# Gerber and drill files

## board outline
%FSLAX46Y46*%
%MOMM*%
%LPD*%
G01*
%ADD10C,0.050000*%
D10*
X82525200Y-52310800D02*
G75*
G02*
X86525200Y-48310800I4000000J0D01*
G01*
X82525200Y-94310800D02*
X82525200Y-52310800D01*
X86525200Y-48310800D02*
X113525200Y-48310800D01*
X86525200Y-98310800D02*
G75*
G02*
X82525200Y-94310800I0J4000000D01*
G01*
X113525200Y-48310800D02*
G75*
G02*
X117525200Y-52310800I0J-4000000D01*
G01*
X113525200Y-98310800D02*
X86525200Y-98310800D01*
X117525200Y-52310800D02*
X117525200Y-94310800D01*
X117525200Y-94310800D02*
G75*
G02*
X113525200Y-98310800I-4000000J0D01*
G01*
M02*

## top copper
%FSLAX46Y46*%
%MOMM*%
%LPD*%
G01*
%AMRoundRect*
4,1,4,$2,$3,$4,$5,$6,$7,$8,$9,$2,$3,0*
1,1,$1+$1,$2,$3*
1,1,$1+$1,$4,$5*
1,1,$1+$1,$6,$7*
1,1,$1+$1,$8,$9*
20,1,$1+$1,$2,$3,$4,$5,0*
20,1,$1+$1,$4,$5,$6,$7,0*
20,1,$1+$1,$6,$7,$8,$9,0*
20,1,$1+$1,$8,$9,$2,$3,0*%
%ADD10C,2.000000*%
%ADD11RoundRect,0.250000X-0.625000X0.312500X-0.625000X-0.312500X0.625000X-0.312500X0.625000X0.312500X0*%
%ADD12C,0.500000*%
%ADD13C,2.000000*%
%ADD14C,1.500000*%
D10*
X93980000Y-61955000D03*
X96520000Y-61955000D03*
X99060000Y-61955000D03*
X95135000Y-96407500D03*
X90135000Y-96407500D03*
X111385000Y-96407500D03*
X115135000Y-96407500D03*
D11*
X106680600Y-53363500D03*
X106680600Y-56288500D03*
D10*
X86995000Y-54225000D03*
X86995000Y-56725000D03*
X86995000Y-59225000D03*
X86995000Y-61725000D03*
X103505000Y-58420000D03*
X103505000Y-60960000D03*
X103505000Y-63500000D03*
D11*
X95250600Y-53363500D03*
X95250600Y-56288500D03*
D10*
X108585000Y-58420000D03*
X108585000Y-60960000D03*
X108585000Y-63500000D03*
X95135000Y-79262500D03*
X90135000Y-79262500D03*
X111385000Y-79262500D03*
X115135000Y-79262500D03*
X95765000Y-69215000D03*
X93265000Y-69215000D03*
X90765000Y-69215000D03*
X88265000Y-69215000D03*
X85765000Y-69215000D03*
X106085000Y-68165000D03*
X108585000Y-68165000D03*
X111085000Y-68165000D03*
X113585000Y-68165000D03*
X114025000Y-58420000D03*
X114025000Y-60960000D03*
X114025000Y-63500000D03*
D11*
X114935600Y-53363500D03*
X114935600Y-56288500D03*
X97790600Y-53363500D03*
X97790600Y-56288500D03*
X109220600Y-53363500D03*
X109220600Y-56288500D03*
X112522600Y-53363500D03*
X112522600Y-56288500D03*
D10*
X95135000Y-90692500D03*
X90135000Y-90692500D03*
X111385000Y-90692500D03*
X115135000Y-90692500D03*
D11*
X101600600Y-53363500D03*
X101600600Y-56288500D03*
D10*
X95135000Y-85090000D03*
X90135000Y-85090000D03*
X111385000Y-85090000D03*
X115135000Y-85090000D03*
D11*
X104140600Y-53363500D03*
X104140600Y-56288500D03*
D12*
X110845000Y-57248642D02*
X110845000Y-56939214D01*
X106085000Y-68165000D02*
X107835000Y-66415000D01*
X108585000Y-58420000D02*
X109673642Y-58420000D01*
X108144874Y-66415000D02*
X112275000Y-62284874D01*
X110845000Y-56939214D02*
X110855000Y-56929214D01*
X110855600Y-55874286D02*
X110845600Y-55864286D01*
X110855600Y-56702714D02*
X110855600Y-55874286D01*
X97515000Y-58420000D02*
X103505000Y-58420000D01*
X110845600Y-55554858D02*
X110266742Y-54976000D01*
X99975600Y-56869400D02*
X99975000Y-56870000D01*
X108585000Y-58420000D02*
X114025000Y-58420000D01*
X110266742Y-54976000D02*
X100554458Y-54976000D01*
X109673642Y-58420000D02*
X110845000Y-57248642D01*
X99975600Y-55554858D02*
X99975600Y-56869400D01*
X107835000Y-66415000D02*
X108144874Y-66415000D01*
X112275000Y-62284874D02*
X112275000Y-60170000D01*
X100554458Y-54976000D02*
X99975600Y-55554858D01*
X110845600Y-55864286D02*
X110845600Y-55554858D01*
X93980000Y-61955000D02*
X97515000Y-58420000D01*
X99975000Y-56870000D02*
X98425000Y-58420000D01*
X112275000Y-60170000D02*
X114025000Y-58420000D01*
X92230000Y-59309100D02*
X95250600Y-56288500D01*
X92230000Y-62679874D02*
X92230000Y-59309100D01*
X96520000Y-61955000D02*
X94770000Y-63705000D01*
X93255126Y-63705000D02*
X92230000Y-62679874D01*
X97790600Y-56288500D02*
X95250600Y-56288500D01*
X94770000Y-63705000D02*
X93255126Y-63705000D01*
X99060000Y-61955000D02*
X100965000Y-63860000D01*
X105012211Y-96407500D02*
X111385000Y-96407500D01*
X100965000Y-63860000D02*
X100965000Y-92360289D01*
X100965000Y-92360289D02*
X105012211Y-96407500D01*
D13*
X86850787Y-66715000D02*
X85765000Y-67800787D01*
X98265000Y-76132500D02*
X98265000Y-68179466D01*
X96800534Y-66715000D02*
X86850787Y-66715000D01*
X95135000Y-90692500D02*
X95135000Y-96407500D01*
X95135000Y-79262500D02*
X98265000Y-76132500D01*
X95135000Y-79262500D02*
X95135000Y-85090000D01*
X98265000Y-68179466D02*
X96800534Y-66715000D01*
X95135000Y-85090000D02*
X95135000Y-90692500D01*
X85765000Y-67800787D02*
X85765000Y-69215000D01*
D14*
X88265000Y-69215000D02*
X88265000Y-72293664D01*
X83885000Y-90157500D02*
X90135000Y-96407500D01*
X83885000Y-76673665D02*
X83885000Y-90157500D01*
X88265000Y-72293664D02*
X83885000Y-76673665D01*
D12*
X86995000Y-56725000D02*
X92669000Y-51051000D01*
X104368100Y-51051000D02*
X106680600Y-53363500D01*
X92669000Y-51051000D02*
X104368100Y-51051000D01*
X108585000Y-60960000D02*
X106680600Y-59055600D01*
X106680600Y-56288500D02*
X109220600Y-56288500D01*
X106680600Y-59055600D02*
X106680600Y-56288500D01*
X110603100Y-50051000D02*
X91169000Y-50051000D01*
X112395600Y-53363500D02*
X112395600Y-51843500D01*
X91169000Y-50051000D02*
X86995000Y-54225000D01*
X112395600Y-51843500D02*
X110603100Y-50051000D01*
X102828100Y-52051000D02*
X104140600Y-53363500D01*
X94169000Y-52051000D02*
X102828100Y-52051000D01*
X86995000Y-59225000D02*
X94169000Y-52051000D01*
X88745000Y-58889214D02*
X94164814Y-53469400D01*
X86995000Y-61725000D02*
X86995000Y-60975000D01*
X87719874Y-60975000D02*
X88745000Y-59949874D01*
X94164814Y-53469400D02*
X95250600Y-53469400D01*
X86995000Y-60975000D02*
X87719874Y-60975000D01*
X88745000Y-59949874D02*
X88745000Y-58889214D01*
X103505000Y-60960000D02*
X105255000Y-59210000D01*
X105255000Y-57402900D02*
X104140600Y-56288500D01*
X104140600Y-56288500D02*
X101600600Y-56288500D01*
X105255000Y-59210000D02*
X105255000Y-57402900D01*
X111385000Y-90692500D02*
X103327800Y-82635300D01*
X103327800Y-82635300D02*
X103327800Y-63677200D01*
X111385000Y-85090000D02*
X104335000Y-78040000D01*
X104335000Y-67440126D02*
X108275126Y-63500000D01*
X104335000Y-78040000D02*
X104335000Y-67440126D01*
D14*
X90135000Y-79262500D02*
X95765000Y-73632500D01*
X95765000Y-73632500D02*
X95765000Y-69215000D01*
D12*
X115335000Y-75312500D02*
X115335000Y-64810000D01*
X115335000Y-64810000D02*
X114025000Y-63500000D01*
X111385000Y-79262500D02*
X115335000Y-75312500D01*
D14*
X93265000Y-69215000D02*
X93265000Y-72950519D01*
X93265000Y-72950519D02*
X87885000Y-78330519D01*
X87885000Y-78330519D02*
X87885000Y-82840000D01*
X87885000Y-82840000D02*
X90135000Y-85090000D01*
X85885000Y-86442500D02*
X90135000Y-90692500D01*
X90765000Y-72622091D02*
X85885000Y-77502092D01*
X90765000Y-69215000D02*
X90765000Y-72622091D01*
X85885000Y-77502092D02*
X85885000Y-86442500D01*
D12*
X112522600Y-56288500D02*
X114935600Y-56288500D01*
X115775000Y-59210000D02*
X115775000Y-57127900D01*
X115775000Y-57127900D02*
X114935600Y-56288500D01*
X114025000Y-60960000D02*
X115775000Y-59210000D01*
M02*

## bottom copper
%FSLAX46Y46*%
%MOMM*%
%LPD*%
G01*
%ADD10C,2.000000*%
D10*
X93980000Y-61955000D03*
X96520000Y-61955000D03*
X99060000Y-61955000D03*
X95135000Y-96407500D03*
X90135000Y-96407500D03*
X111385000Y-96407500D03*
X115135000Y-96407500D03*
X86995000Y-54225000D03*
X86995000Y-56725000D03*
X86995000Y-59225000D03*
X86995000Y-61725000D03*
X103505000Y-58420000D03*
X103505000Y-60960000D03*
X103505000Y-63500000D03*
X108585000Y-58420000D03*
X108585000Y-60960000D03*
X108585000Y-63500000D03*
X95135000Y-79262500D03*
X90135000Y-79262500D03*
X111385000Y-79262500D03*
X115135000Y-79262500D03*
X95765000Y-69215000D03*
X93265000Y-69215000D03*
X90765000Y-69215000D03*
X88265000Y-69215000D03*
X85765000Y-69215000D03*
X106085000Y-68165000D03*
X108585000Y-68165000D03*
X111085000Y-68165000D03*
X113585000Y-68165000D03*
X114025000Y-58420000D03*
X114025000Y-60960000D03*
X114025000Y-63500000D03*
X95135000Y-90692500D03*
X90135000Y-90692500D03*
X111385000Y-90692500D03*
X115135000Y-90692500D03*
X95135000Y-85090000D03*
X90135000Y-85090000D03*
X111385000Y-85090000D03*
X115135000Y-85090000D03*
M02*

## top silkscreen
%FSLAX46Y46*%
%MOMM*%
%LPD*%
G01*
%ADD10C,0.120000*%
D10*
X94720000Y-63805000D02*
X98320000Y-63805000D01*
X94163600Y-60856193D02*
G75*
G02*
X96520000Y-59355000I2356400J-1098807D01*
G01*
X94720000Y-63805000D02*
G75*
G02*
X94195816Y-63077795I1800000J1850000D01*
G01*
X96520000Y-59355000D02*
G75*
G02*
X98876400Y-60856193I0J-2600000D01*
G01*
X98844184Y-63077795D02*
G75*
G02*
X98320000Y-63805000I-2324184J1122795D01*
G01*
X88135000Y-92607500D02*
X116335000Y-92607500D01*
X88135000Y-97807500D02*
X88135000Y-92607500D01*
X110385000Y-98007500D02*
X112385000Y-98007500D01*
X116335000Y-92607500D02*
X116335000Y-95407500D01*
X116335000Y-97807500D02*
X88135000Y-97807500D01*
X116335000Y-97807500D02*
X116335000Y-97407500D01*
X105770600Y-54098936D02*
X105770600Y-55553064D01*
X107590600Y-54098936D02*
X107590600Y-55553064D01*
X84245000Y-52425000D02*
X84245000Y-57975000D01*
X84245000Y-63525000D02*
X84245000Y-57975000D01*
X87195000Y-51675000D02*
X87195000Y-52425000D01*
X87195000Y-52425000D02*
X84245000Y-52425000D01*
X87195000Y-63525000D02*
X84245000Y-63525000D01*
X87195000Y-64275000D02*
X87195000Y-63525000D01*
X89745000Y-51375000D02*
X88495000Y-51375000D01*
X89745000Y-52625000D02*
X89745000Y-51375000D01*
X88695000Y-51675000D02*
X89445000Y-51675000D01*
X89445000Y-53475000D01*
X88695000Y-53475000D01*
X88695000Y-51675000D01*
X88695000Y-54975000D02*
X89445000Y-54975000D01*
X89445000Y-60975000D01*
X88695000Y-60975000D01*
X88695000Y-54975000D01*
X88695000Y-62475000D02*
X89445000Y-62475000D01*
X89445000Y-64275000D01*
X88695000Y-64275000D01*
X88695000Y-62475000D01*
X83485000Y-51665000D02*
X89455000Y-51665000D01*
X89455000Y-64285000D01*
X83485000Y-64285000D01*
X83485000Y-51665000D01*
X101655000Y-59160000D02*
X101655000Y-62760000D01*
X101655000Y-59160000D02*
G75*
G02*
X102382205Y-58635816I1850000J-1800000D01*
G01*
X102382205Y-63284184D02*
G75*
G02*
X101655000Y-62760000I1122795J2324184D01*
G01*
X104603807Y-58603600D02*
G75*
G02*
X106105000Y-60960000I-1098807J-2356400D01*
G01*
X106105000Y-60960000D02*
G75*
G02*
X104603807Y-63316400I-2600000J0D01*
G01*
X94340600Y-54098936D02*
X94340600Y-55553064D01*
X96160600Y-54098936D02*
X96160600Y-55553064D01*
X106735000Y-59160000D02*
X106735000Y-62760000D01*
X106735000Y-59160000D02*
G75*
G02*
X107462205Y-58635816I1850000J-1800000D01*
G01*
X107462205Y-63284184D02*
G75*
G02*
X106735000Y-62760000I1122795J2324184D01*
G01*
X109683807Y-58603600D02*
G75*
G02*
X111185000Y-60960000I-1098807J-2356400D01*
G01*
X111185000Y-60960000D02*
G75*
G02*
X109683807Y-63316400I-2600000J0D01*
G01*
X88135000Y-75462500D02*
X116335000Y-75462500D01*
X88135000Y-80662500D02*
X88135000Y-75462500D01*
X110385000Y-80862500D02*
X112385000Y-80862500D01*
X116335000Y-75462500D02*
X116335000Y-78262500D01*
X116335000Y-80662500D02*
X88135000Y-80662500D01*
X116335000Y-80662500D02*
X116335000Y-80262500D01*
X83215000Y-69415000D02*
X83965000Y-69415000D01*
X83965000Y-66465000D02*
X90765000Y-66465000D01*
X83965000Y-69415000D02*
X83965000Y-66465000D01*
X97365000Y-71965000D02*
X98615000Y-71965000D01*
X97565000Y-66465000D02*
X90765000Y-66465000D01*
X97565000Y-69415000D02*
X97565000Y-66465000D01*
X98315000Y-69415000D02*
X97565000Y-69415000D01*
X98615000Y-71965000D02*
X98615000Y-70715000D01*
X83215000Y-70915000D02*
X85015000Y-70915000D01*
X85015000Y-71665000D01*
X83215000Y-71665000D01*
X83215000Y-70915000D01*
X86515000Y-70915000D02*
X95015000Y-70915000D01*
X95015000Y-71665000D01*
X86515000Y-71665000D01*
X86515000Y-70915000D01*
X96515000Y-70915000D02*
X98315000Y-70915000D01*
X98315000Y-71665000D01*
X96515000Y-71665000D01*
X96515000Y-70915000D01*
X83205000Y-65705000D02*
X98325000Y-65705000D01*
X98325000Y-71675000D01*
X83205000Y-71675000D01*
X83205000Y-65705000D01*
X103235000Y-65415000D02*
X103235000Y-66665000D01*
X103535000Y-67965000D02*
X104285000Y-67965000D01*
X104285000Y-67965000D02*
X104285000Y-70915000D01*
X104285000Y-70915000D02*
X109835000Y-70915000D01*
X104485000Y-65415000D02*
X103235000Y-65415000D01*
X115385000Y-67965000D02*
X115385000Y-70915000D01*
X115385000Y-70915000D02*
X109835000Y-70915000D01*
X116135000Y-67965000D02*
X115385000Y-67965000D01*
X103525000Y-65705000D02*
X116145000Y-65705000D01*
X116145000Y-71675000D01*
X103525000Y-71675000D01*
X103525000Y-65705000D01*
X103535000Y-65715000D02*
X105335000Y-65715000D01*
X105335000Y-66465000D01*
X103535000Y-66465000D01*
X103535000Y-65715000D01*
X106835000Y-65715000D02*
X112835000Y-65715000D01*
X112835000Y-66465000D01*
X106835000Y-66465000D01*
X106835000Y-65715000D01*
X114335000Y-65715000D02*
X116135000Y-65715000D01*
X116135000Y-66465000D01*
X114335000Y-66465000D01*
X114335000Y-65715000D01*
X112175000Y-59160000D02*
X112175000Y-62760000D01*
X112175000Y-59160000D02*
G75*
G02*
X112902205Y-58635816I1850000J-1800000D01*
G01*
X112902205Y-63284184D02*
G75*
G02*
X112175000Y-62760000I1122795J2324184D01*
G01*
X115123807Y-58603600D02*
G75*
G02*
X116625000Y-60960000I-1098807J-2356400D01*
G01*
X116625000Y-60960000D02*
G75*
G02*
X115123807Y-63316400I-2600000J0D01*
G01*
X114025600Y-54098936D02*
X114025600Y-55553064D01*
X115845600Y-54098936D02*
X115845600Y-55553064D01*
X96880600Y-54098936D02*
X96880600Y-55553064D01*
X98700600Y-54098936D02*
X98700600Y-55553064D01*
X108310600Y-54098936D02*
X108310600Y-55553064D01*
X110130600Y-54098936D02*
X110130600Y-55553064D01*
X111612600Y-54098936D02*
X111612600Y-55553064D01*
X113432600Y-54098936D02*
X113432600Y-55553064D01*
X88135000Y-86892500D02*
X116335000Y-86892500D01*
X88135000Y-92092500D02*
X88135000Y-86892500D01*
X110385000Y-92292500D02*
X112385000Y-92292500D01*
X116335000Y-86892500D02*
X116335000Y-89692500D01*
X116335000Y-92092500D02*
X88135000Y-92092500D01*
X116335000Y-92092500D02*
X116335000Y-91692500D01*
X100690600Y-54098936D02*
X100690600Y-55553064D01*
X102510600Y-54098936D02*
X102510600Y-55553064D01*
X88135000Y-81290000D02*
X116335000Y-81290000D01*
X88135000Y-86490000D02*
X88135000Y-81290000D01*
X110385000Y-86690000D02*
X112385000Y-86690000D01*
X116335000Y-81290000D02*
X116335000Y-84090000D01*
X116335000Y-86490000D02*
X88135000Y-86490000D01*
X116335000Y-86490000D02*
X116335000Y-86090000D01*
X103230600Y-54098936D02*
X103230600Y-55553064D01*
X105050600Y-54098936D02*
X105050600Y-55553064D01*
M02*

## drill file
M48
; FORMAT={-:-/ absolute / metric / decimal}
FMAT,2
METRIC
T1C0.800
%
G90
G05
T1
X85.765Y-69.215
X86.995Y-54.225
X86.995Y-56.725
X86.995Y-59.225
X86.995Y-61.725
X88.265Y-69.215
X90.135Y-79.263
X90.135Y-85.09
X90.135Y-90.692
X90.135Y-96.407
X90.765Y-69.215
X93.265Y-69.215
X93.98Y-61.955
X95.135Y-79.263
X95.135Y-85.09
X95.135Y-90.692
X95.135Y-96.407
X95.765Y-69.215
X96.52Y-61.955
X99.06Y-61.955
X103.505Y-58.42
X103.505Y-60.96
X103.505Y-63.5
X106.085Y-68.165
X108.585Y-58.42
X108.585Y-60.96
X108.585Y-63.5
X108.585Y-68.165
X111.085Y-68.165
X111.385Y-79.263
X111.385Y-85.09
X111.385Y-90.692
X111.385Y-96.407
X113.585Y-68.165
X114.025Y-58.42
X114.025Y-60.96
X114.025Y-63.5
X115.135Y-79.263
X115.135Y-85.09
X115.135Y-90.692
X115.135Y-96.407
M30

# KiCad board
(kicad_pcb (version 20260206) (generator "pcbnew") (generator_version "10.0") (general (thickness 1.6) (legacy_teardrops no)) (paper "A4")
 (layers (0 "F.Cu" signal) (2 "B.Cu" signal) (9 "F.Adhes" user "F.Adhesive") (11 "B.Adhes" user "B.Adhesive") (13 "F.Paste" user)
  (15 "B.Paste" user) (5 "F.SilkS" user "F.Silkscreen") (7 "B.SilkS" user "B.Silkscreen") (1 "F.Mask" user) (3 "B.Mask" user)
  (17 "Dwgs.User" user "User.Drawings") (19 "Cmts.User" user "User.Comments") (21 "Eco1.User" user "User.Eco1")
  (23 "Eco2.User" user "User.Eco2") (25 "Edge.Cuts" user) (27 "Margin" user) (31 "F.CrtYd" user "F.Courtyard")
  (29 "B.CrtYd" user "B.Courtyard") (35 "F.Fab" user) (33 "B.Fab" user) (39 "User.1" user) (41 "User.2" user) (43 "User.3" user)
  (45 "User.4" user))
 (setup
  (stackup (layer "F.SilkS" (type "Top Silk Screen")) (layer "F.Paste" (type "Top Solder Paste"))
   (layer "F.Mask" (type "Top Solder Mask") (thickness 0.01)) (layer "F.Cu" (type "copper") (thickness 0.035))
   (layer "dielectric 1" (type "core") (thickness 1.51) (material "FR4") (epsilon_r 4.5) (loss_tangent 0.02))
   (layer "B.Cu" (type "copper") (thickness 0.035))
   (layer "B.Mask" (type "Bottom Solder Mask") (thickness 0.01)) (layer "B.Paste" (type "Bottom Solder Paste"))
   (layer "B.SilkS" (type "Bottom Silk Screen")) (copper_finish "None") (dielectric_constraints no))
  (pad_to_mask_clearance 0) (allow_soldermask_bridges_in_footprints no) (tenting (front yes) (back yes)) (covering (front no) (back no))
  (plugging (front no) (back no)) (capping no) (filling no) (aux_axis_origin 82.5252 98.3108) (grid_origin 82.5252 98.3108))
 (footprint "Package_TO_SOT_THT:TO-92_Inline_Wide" (layer "F.Cu") (at 93.98 61.955)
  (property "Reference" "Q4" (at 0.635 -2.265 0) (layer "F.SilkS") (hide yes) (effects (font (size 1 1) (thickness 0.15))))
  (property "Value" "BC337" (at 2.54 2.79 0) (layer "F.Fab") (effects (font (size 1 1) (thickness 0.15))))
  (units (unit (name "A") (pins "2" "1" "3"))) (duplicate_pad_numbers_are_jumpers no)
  (fp_line (start 0.74 1.85) (end 4.34 1.85) (stroke (width 0.12) (type solid)) (layer "F.SilkS"))
  (fp_arc (start 0.1836 -1.098807) (mid 1.143021 -2.192817) (end 2.54 -2.6) (stroke (width 0.12) (type solid)) (layer "F.SilkS"))
  (fp_arc (start 0.74 1.85) (mid 0.446097 1.509328) (end 0.215816 1.122795) (stroke (width 0.12) (type solid)) (layer "F.SilkS"))
  (fp_arc (start 2.54 -2.6) (mid 3.936979 -2.192818) (end 4.8964 -1.098807) (stroke (width 0.12) (type solid)) (layer "F.SilkS"))
  (fp_arc (start 4.864184 1.122795) (mid 4.633903 1.509328) (end 4.34 1.85) (stroke (width 0.12) (type solid)) (layer "F.SilkS"))
  (pad "1" thru_hole circle (at 0 0) (size 2 1.5) (drill 0.8) (layers "*.Cu" "*.Mask") (remove_unused_layers no) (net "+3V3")
   (thermal_bridge_angle 90))
  (pad "2" thru_hole circle (at 2.54 0) (size 2 1.5) (drill 0.8) (layers "*.Cu" "*.Mask") (remove_unused_layers no) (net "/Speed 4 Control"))
  (pad "3" thru_hole circle (at 5.08 0) (size 2 1.5) (drill 0.8) (layers "*.Cu" "*.Mask") (remove_unused_layers no) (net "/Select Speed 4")))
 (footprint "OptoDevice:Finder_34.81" (layer "F.Cu") (at 111.385 96.4075 180)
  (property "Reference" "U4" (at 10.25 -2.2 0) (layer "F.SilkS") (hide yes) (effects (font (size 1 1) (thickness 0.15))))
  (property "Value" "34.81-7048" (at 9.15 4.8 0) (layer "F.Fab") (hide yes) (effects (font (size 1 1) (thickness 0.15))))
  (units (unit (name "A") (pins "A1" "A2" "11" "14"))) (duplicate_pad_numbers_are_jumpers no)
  (fp_line (start 23.25 3.8) (end -4.95 3.8) (stroke (width 0.12) (type solid)) (layer "F.SilkS"))
  (fp_line (start 23.25 -1.4) (end 23.25 3.8) (stroke (width 0.12) (type solid)) (layer "F.SilkS"))
  (fp_line (start 1 -1.6) (end -1 -1.6) (stroke (width 0.12) (type solid)) (layer "F.SilkS"))
  (fp_line (start -4.95 3.8) (end -4.95 1) (stroke (width 0.12) (type solid)) (layer "F.SilkS"))
  (fp_line (start -4.95 -1.4) (end 23.25 -1.4) (stroke (width 0.12) (type solid)) (layer "F.SilkS"))
  (fp_line (start -4.95 -1.4) (end -4.95 -1) (stroke (width 0.12) (type solid)) (layer "F.SilkS"))
  (pad "11" thru_hole circle (at 16.25 0 180) (size 2 2.4) (drill 0.8) (layers "*.Cu" "*.Mask") (remove_unused_layers no) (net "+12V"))
  (pad "14" thru_hole circle (at 21.25 0 180) (size 2 2.4) (drill 0.8) (layers "*.Cu" "*.Mask") (remove_unused_layers no) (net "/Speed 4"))
  (pad "A1" thru_hole circle (at 0 0 180) (size 2 2.4) (drill 0.8) (layers "*.Cu" "*.Mask") (remove_unused_layers no)
   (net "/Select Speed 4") (thermal_bridge_angle 90))
  (pad "A2" thru_hole circle (at -3.75 0 180) (size 2 2.4) (drill 0.8) (layers "*.Cu" "*.Mask") (remove_unused_layers no) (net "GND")))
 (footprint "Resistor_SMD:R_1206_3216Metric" (layer "F.Cu") (at 106.6806 54.826 -90)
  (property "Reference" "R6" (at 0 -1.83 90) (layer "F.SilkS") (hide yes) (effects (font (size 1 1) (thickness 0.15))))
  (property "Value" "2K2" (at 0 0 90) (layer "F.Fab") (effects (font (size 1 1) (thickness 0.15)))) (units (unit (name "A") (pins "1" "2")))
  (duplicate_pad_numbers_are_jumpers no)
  (fp_line (start -0.727064 0.91) (end 0.727064 0.91) (stroke (width 0.12) (type solid)) (layer "F.SilkS"))
  (fp_line (start -0.727064 -0.91) (end 0.727064 -0.91) (stroke (width 0.12) (type solid)) (layer "F.SilkS"))
  (pad "1" smd roundrect (at -1.4625 0 270) (size 1.125 1.75) (layers "F.Cu" "F.Mask" "F.Paste") (roundrect_rratio 0.222222) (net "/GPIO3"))
  (pad "2" smd roundrect (at 1.4625 0 270) (size 1.125 1.75) (layers "F.Cu" "F.Mask" "F.Paste") (roundrect_rratio 0.222222)
   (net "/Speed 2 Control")))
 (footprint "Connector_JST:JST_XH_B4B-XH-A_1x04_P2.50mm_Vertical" (layer "F.Cu") (at 86.995 54.225 -90)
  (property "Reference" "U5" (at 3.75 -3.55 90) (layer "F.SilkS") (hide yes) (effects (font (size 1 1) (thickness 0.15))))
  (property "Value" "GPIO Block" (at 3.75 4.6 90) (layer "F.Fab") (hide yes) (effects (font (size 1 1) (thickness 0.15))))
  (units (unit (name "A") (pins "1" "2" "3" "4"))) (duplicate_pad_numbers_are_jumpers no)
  (fp_line (start -1.8 2.75) (end 3.75 2.75) (stroke (width 0.12) (type solid)) (layer "F.SilkS"))
  (fp_line (start 9.3 2.75) (end 3.75 2.75) (stroke (width 0.12) (type solid)) (layer "F.SilkS"))
  (fp_line (start -2.55 -0.2) (end -1.8 -0.2) (stroke (width 0.12) (type solid)) (layer "F.SilkS"))
  (fp_line (start -1.8 -0.2) (end -1.8 2.75) (stroke (width 0.12) (type solid)) (layer "F.SilkS"))
  (fp_line (start 9.3 -0.2) (end 9.3 2.75) (stroke (width 0.12) (type solid)) (layer "F.SilkS"))
  (fp_line (start 10.05 -0.2) (end 9.3 -0.2) (stroke (width 0.12) (type solid)) (layer "F.SilkS"))
  (fp_line (start -2.85 -2.75) (end -2.85 -1.5) (stroke (width 0.12) (type solid)) (layer "F.SilkS"))
  (fp_line (start -1.6 -2.75) (end -2.85 -2.75) (stroke (width 0.12) (type solid)) (layer "F.SilkS"))
  (fp_rect (start -2.55 -2.45) (end -0.75 -1.7) (stroke (width 0.12) (type solid)) (fill no) (layer "F.SilkS"))
  (fp_rect (start 0.75 -2.45) (end 6.75 -1.7) (stroke (width 0.12) (type solid)) (fill no) (layer "F.SilkS"))
  (fp_rect (start 8.25 -2.45) (end 10.05 -1.7) (stroke (width 0.12) (type solid)) (fill no) (layer "F.SilkS"))
  (fp_rect (start -2.56 -2.46) (end 10.06 3.51) (stroke (width 0.12) (type solid)) (fill no) (layer "F.SilkS"))
  (pad "1" thru_hole circle (at 0 0 270) (size 2 1.95) (drill 0.8) (layers "*.Cu" "*.Mask") (remove_unused_layers no) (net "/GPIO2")
   (thermal_bridge_angle 90))
  (pad "2" thru_hole circle (at 2.5 0 270) (size 2 1.95) (drill 0.8) (layers "*.Cu" "*.Mask") (remove_unused_layers no) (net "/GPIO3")
   (thermal_bridge_angle 90))
  (pad "3" thru_hole circle (at 5 0 270) (size 2 1.95) (drill 0.8) (layers "*.Cu" "*.Mask") (remove_unused_layers no) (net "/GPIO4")
   (thermal_bridge_angle 90))
  (pad "4" thru_hole circle (at 7.5 0 270) (size 2 1.95) (drill 0.8) (layers "*.Cu" "*.Mask") (remove_unused_layers no) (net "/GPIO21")
   (thermal_bridge_angle 90)))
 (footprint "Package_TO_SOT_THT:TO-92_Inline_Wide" (layer "F.Cu") (at 103.505 58.42 -90)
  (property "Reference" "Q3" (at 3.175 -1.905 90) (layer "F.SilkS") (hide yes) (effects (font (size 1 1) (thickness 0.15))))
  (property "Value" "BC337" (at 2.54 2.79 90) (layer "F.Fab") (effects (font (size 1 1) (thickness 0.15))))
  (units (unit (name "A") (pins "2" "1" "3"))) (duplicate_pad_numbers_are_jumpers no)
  (fp_line (start 0.74 1.85) (end 4.34 1.85) (stroke (width 0.12) (type solid)) (layer "F.SilkS"))
  (fp_arc (start 0.74 1.85) (mid 0.446097 1.509328) (end 0.215816 1.122795) (stroke (width 0.12) (type solid)) (layer "F.SilkS"))
  (fp_arc (start 4.864184 1.122795) (mid 4.633903 1.509328) (end 4.34 1.85) (stroke (width 0.12) (type solid)) (layer "F.SilkS"))
  (fp_arc (start 0.1836 -1.098807) (mid 1.143021 -2.192817) (end 2.54 -2.6) (stroke (width 0.12) (type solid)) (layer "F.SilkS"))
  (fp_arc (start 2.54 -2.6) (mid 3.936979 -2.192818) (end 4.8964 -1.098807) (stroke (width 0.12) (type solid)) (layer "F.SilkS"))
  (pad "1" thru_hole circle (at 0 0 270) (size 2 1.5) (drill 0.8) (layers "*.Cu" "*.Mask") (remove_unused_layers no) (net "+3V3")
   (thermal_bridge_angle 90))
  (pad "2" thru_hole circle (at 2.54 0 270) (size 2 1.5) (drill 0.8) (layers "*.Cu" "*.Mask") (remove_unused_layers no)
   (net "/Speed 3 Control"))
  (pad "3" thru_hole circle (at 5.08 0 270) (size 2 1.5) (drill 0.8) (layers "*.Cu" "*.Mask") (remove_unused_layers no)
   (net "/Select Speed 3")))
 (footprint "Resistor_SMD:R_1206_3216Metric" (layer "F.Cu") (at 95.2506 54.826 -90)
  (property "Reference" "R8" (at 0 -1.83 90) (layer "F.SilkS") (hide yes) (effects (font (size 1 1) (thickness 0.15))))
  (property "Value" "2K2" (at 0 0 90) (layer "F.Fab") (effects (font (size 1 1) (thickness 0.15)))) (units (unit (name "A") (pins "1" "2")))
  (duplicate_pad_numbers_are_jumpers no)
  (fp_line (start -0.727064 0.91) (end 0.727064 0.91) (stroke (width 0.12) (type solid)) (layer "F.SilkS"))
  (fp_line (start -0.727064 -0.91) (end 0.727064 -0.91) (stroke (width 0.12) (type solid)) (layer "F.SilkS"))
  (pad "1" smd roundrect (at -1.4625 0 270) (size 1.125 1.75) (layers "F.Cu" "F.Mask" "F.Paste") (roundrect_rratio 0.222222) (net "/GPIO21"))
  (pad "2" smd roundrect (at 1.4625 0 270) (size 1.125 1.75) (layers "F.Cu" "F.Mask" "F.Paste") (roundrect_rratio 0.222222)
   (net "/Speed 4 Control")))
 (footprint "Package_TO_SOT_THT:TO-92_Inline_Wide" (layer "F.Cu") (at 108.585 58.42 -90)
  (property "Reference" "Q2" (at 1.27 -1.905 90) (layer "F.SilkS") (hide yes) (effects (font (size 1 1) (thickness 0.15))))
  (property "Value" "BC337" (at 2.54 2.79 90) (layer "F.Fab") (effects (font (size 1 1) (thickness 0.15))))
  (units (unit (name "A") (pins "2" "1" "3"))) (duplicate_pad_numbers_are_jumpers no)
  (fp_line (start 0.74 1.85) (end 4.34 1.85) (stroke (width 0.12) (type solid)) (layer "F.SilkS"))
  (fp_arc (start 0.74 1.85) (mid 0.446097 1.509328) (end 0.215816 1.122795) (stroke (width 0.12) (type solid)) (layer "F.SilkS"))
  (fp_arc (start 4.864184 1.122795) (mid 4.633903 1.509328) (end 4.34 1.85) (stroke (width 0.12) (type solid)) (layer "F.SilkS"))
  (fp_arc (start 0.1836 -1.098807) (mid 1.143021 -2.192817) (end 2.54 -2.6) (stroke (width 0.12) (type solid)) (layer "F.SilkS"))
  (fp_arc (start 2.54 -2.6) (mid 3.936979 -2.192818) (end 4.8964 -1.098807) (stroke (width 0.12) (type solid)) (layer "F.SilkS"))
  (pad "1" thru_hole circle (at 0 0 270) (size 2 1.5) (drill 0.8) (layers "*.Cu" "*.Mask") (remove_unused_layers no) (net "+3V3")
   (thermal_bridge_angle 90))
  (pad "2" thru_hole circle (at 2.54 0 270) (size 2 1.5) (drill 0.8) (layers "*.Cu" "*.Mask") (remove_unused_layers no)
   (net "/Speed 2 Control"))
  (pad "3" thru_hole circle (at 5.08 0 270) (size 2 1.5) (drill 0.8) (layers "*.Cu" "*.Mask") (remove_unused_layers no)
   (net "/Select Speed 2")))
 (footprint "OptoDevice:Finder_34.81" (layer "F.Cu") (at 111.385 79.2625 180)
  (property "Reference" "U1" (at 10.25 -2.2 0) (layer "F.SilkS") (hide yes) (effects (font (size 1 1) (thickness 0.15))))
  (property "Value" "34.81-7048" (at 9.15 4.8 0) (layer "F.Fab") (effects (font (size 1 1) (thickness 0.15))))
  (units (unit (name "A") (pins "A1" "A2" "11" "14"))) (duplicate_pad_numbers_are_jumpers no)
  (fp_line (start 23.25 3.8) (end -4.95 3.8) (stroke (width 0.12) (type solid)) (layer "F.SilkS"))
  (fp_line (start 23.25 -1.4) (end 23.25 3.8) (stroke (width 0.12) (type solid)) (layer "F.SilkS"))
  (fp_line (start 1 -1.6) (end -1 -1.6) (stroke (width 0.12) (type solid)) (layer "F.SilkS"))
  (fp_line (start -4.95 3.8) (end -4.95 1) (stroke (width 0.12) (type solid)) (layer "F.SilkS"))
  (fp_line (start -4.95 -1.4) (end 23.25 -1.4) (stroke (width 0.12) (type solid)) (layer "F.SilkS"))
  (fp_line (start -4.95 -1.4) (end -4.95 -1) (stroke (width 0.12) (type solid)) (layer "F.SilkS"))
  (pad "11" thru_hole circle (at 16.25 0 180) (size 2 2.4) (drill 0.8) (layers "*.Cu" "*.Mask") (remove_unused_layers no) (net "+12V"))
  (pad "14" thru_hole circle (at 21.25 0 180) (size 2 2.4) (drill 0.8) (layers "*.Cu" "*.Mask") (remove_unused_layers no) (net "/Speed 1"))
  (pad "A1" thru_hole circle (at 0 0 180) (size 2 2.4) (drill 0.8) (layers "*.Cu" "*.Mask") (remove_unused_layers no)
   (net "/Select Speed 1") (thermal_bridge_angle 90))
  (pad "A2" thru_hole circle (at -3.75 0 180) (size 2 2.4) (drill 0.8) (layers "*.Cu" "*.Mask") (remove_unused_layers no) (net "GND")))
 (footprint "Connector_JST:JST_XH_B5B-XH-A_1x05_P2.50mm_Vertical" (layer "F.Cu") (at 95.765 69.215 180)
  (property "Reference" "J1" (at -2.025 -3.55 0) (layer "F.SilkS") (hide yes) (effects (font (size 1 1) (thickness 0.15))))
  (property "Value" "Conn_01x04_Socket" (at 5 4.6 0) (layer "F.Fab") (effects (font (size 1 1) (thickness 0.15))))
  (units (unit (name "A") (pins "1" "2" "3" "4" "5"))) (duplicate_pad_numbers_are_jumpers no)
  (fp_line (start 12.55 -0.2) (end 11.8 -0.2) (stroke (width 0.12) (type solid)) (layer "F.SilkS"))
  (fp_line (start 11.8 2.75) (end 5 2.75) (stroke (width 0.12) (type solid)) (layer "F.SilkS"))
  (fp_line (start 11.8 -0.2) (end 11.8 2.75) (stroke (width 0.12) (type solid)) (layer "F.SilkS"))
  (fp_line (start -1.6 -2.75) (end -2.85 -2.75) (stroke (width 0.12) (type solid)) (layer "F.SilkS"))
  (fp_line (start -1.8 2.75) (end 5 2.75) (stroke (width 0.12) (type solid)) (layer "F.SilkS"))
  (fp_line (start -1.8 -0.2) (end -1.8 2.75) (stroke (width 0.12) (type solid)) (layer "F.SilkS"))
  (fp_line (start -2.55 -0.2) (end -1.8 -0.2) (stroke (width 0.12) (type solid)) (layer "F.SilkS"))
  (fp_line (start -2.85 -2.75) (end -2.85 -1.5) (stroke (width 0.12) (type solid)) (layer "F.SilkS"))
  (fp_rect (start 10.75 -2.45) (end 12.55 -1.7) (stroke (width 0.12) (type solid)) (fill no) (layer "F.SilkS"))
  (fp_rect (start 0.75 -2.45) (end 9.25 -1.7) (stroke (width 0.12) (type solid)) (fill no) (layer "F.SilkS"))
  (fp_rect (start -2.55 -2.45) (end -0.75 -1.7) (stroke (width 0.12) (type solid)) (fill no) (layer "F.SilkS"))
  (fp_rect (start -2.56 -2.46) (end 12.56 3.51) (stroke (width 0.12) (type solid)) (fill no) (layer "F.SilkS"))
  (pad "1" thru_hole circle (at 0 0 180) (size 2 1.95) (drill 0.8) (layers "*.Cu" "*.Mask") (remove_unused_layers no) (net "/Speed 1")
   (thermal_bridge_angle 90))
  (pad "2" thru_hole circle (at 2.5 0 180) (size 2 1.95) (drill 0.8) (layers "*.Cu" "*.Mask") (remove_unused_layers no) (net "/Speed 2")
   (thermal_bridge_angle 90))
  (pad "3" thru_hole circle (at 5 0 180) (size 2 1.95) (drill 0.8) (layers "*.Cu" "*.Mask") (remove_unused_layers no) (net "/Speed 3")
   (thermal_bridge_angle 90))
  (pad "4" thru_hole circle (at 7.5 0 180) (size 2 1.95) (drill 0.8) (layers "*.Cu" "*.Mask") (remove_unused_layers no) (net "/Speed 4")
   (thermal_bridge_angle 90))
  (pad "5" thru_hole circle (at 10 0 180) (size 2 1.95) (drill 0.8) (layers "*.Cu" "*.Mask") (remove_unused_layers no) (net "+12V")
   (thermal_bridge_angle 90)))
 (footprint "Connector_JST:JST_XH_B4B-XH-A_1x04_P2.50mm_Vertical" (layer "F.Cu") (at 106.085 68.165)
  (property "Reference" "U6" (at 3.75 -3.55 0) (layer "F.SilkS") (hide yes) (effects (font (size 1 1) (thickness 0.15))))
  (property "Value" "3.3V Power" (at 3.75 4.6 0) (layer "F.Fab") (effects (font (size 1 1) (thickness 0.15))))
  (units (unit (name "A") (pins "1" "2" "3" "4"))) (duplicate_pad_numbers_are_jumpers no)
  (fp_line (start -2.85 -2.75) (end -2.85 -1.5) (stroke (width 0.12) (type solid)) (layer "F.SilkS"))
  (fp_line (start -2.55 -0.2) (end -1.8 -0.2) (stroke (width 0.12) (type solid)) (layer "F.SilkS"))
  (fp_line (start -1.8 -0.2) (end -1.8 2.75) (stroke (width 0.12) (type solid)) (layer "F.SilkS"))
  (fp_line (start -1.8 2.75) (end 3.75 2.75) (stroke (width 0.12) (type solid)) (layer "F.SilkS"))
  (fp_line (start -1.6 -2.75) (end -2.85 -2.75) (stroke (width 0.12) (type solid)) (layer "F.SilkS"))
  (fp_line (start 9.3 -0.2) (end 9.3 2.75) (stroke (width 0.12) (type solid)) (layer "F.SilkS"))
  (fp_line (start 9.3 2.75) (end 3.75 2.75) (stroke (width 0.12) (type solid)) (layer "F.SilkS"))
  (fp_line (start 10.05 -0.2) (end 9.3 -0.2) (stroke (width 0.12) (type solid)) (layer "F.SilkS"))
  (fp_rect (start -2.56 -2.46) (end 10.06 3.51) (stroke (width 0.12) (type solid)) (fill no) (layer "F.SilkS"))
  (fp_rect (start -2.55 -2.45) (end -0.75 -1.7) (stroke (width 0.12) (type solid)) (fill no) (layer "F.SilkS"))
  (fp_rect (start 0.75 -2.45) (end 6.75 -1.7) (stroke (width 0.12) (type solid)) (fill no) (layer "F.SilkS"))
  (fp_rect (start 8.25 -2.45) (end 10.05 -1.7) (stroke (width 0.12) (type solid)) (fill no) (layer "F.SilkS"))
  (pad "1" thru_hole circle (at 0 0) (size 2 1.95) (drill 0.8) (layers "*.Cu" "*.Mask") (remove_unused_layers no) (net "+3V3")
   (thermal_bridge_angle 90))
  (pad "2" thru_hole circle (at 2.5 0) (size 2 1.95) (drill 0.8) (layers "*.Cu" "*.Mask") (remove_unused_layers no) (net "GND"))
  (pad "3" thru_hole circle (at 5 0) (size 2 1.95) (drill 0.8) (layers "*.Cu" "*.Mask") (remove_unused_layers no)
   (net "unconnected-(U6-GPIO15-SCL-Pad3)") (thermal_bridge_angle 90))
  (pad "4" thru_hole circle (at 7.5 0) (size 2 1.95) (drill 0.8) (layers "*.Cu" "*.Mask") (remove_unused_layers no)
   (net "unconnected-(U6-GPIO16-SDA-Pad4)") (thermal_bridge_angle 90)))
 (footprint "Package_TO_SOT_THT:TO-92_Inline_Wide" (layer "F.Cu") (at 114.025 58.42 -90)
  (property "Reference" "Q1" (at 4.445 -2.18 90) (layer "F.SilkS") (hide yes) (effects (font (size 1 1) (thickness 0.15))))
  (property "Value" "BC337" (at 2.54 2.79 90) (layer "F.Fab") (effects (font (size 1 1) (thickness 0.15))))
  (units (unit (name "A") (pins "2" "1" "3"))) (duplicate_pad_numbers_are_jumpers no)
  (fp_line (start 0.74 1.85) (end 4.34 1.85) (stroke (width 0.12) (type solid)) (layer "F.SilkS"))
  (fp_arc (start 0.74 1.85) (mid 0.446097 1.509328) (end 0.215816 1.122795) (stroke (width 0.12) (type solid)) (layer "F.SilkS"))
  (fp_arc (start 4.864184 1.122795) (mid 4.633903 1.509328) (end 4.34 1.85) (stroke (width 0.12) (type solid)) (layer "F.SilkS"))
  (fp_arc (start 0.1836 -1.098807) (mid 1.143021 -2.192817) (end 2.54 -2.6) (stroke (width 0.12) (type solid)) (layer "F.SilkS"))
  (fp_arc (start 2.54 -2.6) (mid 3.936979 -2.192818) (end 4.8964 -1.098807) (stroke (width 0.12) (type solid)) (layer "F.SilkS"))
  (pad "1" thru_hole circle (at 0 0 270) (size 2 1.5) (drill 0.8) (layers "*.Cu" "*.Mask") (remove_unused_layers no) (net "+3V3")
   (thermal_bridge_angle 90))
  (pad "2" thru_hole circle (at 2.54 0 270) (size 2 1.5) (drill 0.8) (layers "*.Cu" "*.Mask") (remove_unused_layers no)
   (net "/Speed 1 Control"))
  (pad "3" thru_hole circle (at 5.08 0 270) (size 2 1.5) (drill 0.8) (layers "*.Cu" "*.Mask") (remove_unused_layers no)
   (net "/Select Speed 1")))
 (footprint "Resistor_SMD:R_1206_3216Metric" (layer "F.Cu") (at 114.9356 54.826 -90)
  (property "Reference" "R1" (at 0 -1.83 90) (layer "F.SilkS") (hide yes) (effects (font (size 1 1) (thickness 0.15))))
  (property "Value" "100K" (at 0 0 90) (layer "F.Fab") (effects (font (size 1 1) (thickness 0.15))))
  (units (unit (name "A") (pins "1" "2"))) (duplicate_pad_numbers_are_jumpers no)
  (fp_line (start -0.727064 0.91) (end 0.727064 0.91) (stroke (width 0.12) (type solid)) (layer "F.SilkS"))
  (fp_line (start -0.727064 -0.91) (end 0.727064 -0.91) (stroke (width 0.12) (type solid)) (layer "F.SilkS"))
  (pad "1" smd roundrect (at -1.4625 0 270) (size 1.125 1.75) (layers "F.Cu" "F.Mask" "F.Paste") (roundrect_rratio 0.222222) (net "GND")
   (thermal_bridge_angle 45))
  (pad "2" smd roundrect (at 1.4625 0 270) (size 1.125 1.75) (layers "F.Cu" "F.Mask" "F.Paste") (roundrect_rratio 0.222222)
   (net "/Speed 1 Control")))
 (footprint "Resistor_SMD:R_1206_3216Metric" (layer "F.Cu") (at 97.7906 54.826 -90)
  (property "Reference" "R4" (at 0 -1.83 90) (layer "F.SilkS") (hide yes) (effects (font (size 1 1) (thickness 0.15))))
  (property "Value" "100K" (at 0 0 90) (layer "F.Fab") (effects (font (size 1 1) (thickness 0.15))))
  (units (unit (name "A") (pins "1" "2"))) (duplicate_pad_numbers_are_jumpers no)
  (fp_line (start -0.727064 0.91) (end 0.727064 0.91) (stroke (width 0.12) (type solid)) (layer "F.SilkS"))
  (fp_line (start -0.727064 -0.91) (end 0.727064 -0.91) (stroke (width 0.12) (type solid)) (layer "F.SilkS"))
  (pad "1" smd roundrect (at -1.4625 0 270) (size 1.125 1.75) (layers "F.Cu" "F.Mask" "F.Paste") (roundrect_rratio 0.222222) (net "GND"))
  (pad "2" smd roundrect (at 1.4625 0 270) (size 1.125 1.75) (layers "F.Cu" "F.Mask" "F.Paste") (roundrect_rratio 0.222222)
   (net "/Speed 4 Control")))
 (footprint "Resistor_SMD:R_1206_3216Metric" (layer "F.Cu") (at 109.2206 54.826 -90)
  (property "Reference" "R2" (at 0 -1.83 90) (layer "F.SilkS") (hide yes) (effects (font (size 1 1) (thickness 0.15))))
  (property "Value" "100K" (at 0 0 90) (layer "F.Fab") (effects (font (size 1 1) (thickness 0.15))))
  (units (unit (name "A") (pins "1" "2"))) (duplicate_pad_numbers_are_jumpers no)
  (fp_line (start -0.727064 0.91) (end 0.727064 0.91) (stroke (width 0.12) (type solid)) (layer "F.SilkS"))
  (fp_line (start -0.727064 -0.91) (end 0.727064 -0.91) (stroke (width 0.12) (type solid)) (layer "F.SilkS"))
  (pad "1" smd roundrect (at -1.4625 0 270) (size 1.125 1.75) (layers "F.Cu" "F.Mask" "F.Paste") (roundrect_rratio 0.222222) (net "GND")
   (thermal_bridge_angle 45))
  (pad "2" smd roundrect (at 1.4625 0 270) (size 1.125 1.75) (layers "F.Cu" "F.Mask" "F.Paste") (roundrect_rratio 0.222222)
   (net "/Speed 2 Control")))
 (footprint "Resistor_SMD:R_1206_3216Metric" (layer "F.Cu") (at 112.5226 54.826 -90)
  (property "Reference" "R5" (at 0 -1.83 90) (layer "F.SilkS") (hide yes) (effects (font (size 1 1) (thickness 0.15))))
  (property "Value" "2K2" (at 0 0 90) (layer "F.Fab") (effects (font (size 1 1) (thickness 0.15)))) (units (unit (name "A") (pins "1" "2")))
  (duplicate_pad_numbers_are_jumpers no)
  (fp_line (start -0.727064 0.91) (end 0.727064 0.91) (stroke (width 0.12) (type solid)) (layer "F.SilkS"))
  (fp_line (start -0.727064 -0.91) (end 0.727064 -0.91) (stroke (width 0.12) (type solid)) (layer "F.SilkS"))
  (pad "1" smd roundrect (at -1.4625 0 270) (size 1.125 1.75) (layers "F.Cu" "F.Mask" "F.Paste") (roundrect_rratio 0.222222) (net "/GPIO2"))
  (pad "2" smd roundrect (at 1.4625 0 270) (size 1.125 1.75) (layers "F.Cu" "F.Mask" "F.Paste") (roundrect_rratio 0.222222)
   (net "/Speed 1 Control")))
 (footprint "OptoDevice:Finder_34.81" (layer "F.Cu") (at 111.385 90.6925 180)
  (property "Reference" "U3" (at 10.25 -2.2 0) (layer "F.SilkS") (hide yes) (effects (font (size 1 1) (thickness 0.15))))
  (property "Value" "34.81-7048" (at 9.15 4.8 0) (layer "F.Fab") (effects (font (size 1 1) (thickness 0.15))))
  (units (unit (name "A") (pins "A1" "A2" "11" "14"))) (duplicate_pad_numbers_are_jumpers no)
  (fp_line (start 23.25 3.8) (end -4.95 3.8) (stroke (width 0.12) (type solid)) (layer "F.SilkS"))
  (fp_line (start 23.25 -1.4) (end 23.25 3.8) (stroke (width 0.12) (type solid)) (layer "F.SilkS"))
  (fp_line (start 1 -1.6) (end -1 -1.6) (stroke (width 0.12) (type solid)) (layer "F.SilkS"))
  (fp_line (start -4.95 3.8) (end -4.95 1) (stroke (width 0.12) (type solid)) (layer "F.SilkS"))
  (fp_line (start -4.95 -1.4) (end 23.25 -1.4) (stroke (width 0.12) (type solid)) (layer "F.SilkS"))
  (fp_line (start -4.95 -1.4) (end -4.95 -1) (stroke (width 0.12) (type solid)) (layer "F.SilkS"))
  (pad "11" thru_hole circle (at 16.25 0 180) (size 2 2.4) (drill 0.8) (layers "*.Cu" "*.Mask") (remove_unused_layers no) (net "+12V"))
  (pad "14" thru_hole circle (at 21.25 0 180) (size 2 2.4) (drill 0.8) (layers "*.Cu" "*.Mask") (remove_unused_layers no) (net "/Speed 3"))
  (pad "A1" thru_hole circle (at 0 0 180) (size 2 2.4) (drill 0.8) (layers "*.Cu" "*.Mask") (remove_unused_layers no)
   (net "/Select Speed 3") (thermal_bridge_angle 90))
  (pad "A2" thru_hole circle (at -3.75 0 180) (size 2 2.4) (drill 0.8) (layers "*.Cu" "*.Mask") (remove_unused_layers no) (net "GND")))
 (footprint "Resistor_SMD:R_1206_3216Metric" (layer "F.Cu") (at 101.6006 54.826 -90)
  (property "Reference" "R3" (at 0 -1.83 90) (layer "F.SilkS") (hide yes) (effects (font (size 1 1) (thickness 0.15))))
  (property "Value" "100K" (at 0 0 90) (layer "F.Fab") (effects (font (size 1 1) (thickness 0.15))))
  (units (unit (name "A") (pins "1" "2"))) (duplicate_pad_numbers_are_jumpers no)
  (fp_line (start -0.727064 0.91) (end 0.727064 0.91) (stroke (width 0.12) (type solid)) (layer "F.SilkS"))
  (fp_line (start -0.727064 -0.91) (end 0.727064 -0.91) (stroke (width 0.12) (type solid)) (layer "F.SilkS"))
  (pad "1" smd roundrect (at -1.4625 0 270) (size 1.125 1.75) (layers "F.Cu" "F.Mask" "F.Paste") (roundrect_rratio 0.222222) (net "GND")
   (zone_connect 2))
  (pad "2" smd roundrect (at 1.4625 0 270) (size 1.125 1.75) (layers "F.Cu" "F.Mask" "F.Paste") (roundrect_rratio 0.222222)
   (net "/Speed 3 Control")))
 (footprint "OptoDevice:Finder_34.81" (layer "F.Cu") (at 111.385 85.09 180)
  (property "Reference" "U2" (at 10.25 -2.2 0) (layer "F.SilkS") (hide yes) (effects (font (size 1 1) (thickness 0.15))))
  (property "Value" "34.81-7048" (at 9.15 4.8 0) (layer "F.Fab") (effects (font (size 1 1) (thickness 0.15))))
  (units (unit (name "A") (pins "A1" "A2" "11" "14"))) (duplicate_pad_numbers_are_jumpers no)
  (fp_line (start 23.25 3.8) (end -4.95 3.8) (stroke (width 0.12) (type solid)) (layer "F.SilkS"))
  (fp_line (start 23.25 -1.4) (end 23.25 3.8) (stroke (width 0.12) (type solid)) (layer "F.SilkS"))
  (fp_line (start 1 -1.6) (end -1 -1.6) (stroke (width 0.12) (type solid)) (layer "F.SilkS"))
  (fp_line (start -4.95 3.8) (end -4.95 1) (stroke (width 0.12) (type solid)) (layer "F.SilkS"))
  (fp_line (start -4.95 -1.4) (end 23.25 -1.4) (stroke (width 0.12) (type solid)) (layer "F.SilkS"))
  (fp_line (start -4.95 -1.4) (end -4.95 -1) (stroke (width 0.12) (type solid)) (layer "F.SilkS"))
  (pad "11" thru_hole circle (at 16.25 0 180) (size 2 2.4) (drill 0.8) (layers "*.Cu" "*.Mask") (remove_unused_layers no) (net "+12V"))
  (pad "14" thru_hole circle (at 21.25 0 180) (size 2 2.4) (drill 0.8) (layers "*.Cu" "*.Mask") (remove_unused_layers no) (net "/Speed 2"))
  (pad "A1" thru_hole circle (at 0 0 180) (size 2 2.4) (drill 0.8) (layers "*.Cu" "*.Mask") (remove_unused_layers no)
   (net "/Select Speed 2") (thermal_bridge_angle 90))
  (pad "A2" thru_hole circle (at -3.75 0 180) (size 2 2.4) (drill 0.8) (layers "*.Cu" "*.Mask") (remove_unused_layers no) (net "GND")))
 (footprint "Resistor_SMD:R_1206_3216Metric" (layer "F.Cu") (at 104.1406 54.826 -90)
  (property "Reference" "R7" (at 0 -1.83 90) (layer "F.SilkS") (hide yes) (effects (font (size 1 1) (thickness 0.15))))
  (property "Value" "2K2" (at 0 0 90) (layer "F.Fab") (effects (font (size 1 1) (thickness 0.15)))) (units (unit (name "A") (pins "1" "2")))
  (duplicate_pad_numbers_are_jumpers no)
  (fp_line (start -0.727064 0.91) (end 0.727064 0.91) (stroke (width 0.12) (type solid)) (layer "F.SilkS"))
  (fp_line (start -0.727064 -0.91) (end 0.727064 -0.91) (stroke (width 0.12) (type solid)) (layer "F.SilkS"))
  (pad "1" smd roundrect (at -1.4625 0 270) (size 1.125 1.75) (layers "F.Cu" "F.Mask" "F.Paste") (roundrect_rratio 0.222222) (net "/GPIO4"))
  (pad "2" smd roundrect (at 1.4625 0 270) (size 1.125 1.75) (layers "F.Cu" "F.Mask" "F.Paste") (roundrect_rratio 0.222222)
   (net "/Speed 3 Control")))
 (gr_arc (start 82.5252 52.3108) (mid 83.696773 49.482373) (end 86.5252 48.3108) (stroke (width 0.05) (type default)) (layer "Edge.Cuts"))
 (gr_line (start 82.5252 94.3108) (end 82.5252 52.3108) (stroke (width 0.05) (type default)) (layer "Edge.Cuts"))
 (gr_line (start 86.5252 48.3108) (end 113.5252 48.3108) (stroke (width 0.05) (type default)) (layer "Edge.Cuts"))
 (gr_arc (start 86.5252 98.3108) (mid 83.696773 97.139227) (end 82.5252 94.3108) (stroke (width 0.05) (type default)) (layer "Edge.Cuts"))
 (gr_arc (start 113.5252 48.3108) (mid 116.353627 49.482373) (end 117.5252 52.3108) (stroke (width 0.05) (type default)) (layer "Edge.Cuts"))
 (gr_line (start 113.5252 98.3108) (end 86.5252 98.3108) (stroke (width 0.05) (type default)) (layer "Edge.Cuts"))
 (gr_line (start 117.5252 52.3108) (end 117.5252 94.3108) (stroke (width 0.05) (type default)) (layer "Edge.Cuts"))
 (gr_arc (start 117.5252 94.3108) (mid 116.353627 97.139227) (end 113.5252 98.3108) (stroke (width 0.05) (type default)) (layer "Edge.Cuts"))
 (segment (start 110.845 57.248642) (end 110.845 56.939214) (width 0.5) (layer "F.Cu") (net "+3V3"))
 (segment (start 106.085 68.165) (end 107.835 66.415) (width 0.5) (layer "F.Cu") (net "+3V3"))
 (segment (start 108.585 58.42) (end 109.673642 58.42) (width 0.5) (layer "F.Cu") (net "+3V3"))
 (segment (start 108.144874 66.415) (end 112.275 62.284874) (width 0.5) (layer "F.Cu") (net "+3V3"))
 (segment (start 110.845 56.939214) (end 110.855 56.929214) (width 0.5) (layer "F.Cu") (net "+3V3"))
 (segment (start 110.8556 55.874286) (end 110.8456 55.864286) (width 0.5) (layer "F.Cu") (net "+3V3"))
 (segment (start 110.8556 56.702714) (end 110.8556 55.874286) (width 0.5) (layer "F.Cu") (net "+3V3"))
 (segment (start 97.515 58.42) (end 103.505 58.42) (width 0.5) (layer "F.Cu") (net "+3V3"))
 (segment (start 110.8456 55.554858) (end 110.266742 54.976) (width 0.5) (layer "F.Cu") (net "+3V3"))
 (segment (start 99.9756 56.8694) (end 99.975 56.87) (width 0.5) (layer "F.Cu") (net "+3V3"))
 (segment (start 108.585 58.42) (end 114.025 58.42) (width 0.5) (layer "F.Cu") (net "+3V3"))
 (segment (start 110.266742 54.976) (end 100.554458 54.976) (width 0.5) (layer "F.Cu") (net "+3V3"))
 (segment (start 109.673642 58.42) (end 110.845 57.248642) (width 0.5) (layer "F.Cu") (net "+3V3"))
 (segment (start 99.9756 55.554858) (end 99.9756 56.8694) (width 0.5) (layer "F.Cu") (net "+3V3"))
 (segment (start 107.835 66.415) (end 108.144874 66.415) (width 0.5) (layer "F.Cu") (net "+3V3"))
 (segment (start 112.275 62.284874) (end 112.275 60.17) (width 0.5) (layer "F.Cu") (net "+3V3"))
 (segment (start 100.554458 54.976) (end 99.9756 55.554858) (width 0.5) (layer "F.Cu") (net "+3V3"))
 (segment (start 110.8456 55.864286) (end 110.8456 55.554858) (width 0.5) (layer "F.Cu") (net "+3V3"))
 (segment (start 93.98 61.955) (end 97.515 58.42) (width 0.5) (layer "F.Cu") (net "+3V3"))
 (segment (start 99.975 56.87) (end 98.425 58.42) (width 0.5) (layer "F.Cu") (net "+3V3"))
 (segment (start 112.275 60.17) (end 114.025 58.42) (width 0.5) (layer "F.Cu") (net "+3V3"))
 (segment (start 92.23 59.3091) (end 95.2506 56.2885) (width 0.5) (layer "F.Cu") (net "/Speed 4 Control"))
 (segment (start 92.23 62.679874) (end 92.23 59.3091) (width 0.5) (layer "F.Cu") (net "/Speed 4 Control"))
 (segment (start 96.52 61.955) (end 94.77 63.705) (width 0.5) (layer "F.Cu") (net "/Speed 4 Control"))
 (segment (start 93.255126 63.705) (end 92.23 62.679874) (width 0.5) (layer "F.Cu") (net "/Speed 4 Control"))
 (segment (start 97.7906 56.2885) (end 95.2506 56.2885) (width 0.5) (layer "F.Cu") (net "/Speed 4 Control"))
 (segment (start 94.77 63.705) (end 93.255126 63.705) (width 0.5) (layer "F.Cu") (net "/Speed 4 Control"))
 (segment (start 99.06 61.955) (end 100.965 63.86) (width 0.5) (layer "F.Cu") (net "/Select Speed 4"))
 (segment (start 105.012211 96.4075) (end 111.385 96.4075) (width 0.5) (layer "F.Cu") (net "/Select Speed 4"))
 (segment (start 100.965 63.86) (end 100.965 92.360289) (width 0.5) (layer "F.Cu") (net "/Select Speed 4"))
 (segment (start 100.965 92.360289) (end 105.012211 96.4075) (width 0.5) (layer "F.Cu") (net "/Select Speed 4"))
 (segment (start 86.850787 66.715) (end 85.765 67.800787) (width 2) (layer "F.Cu") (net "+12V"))
 (segment (start 98.265 76.1325) (end 98.265 68.179466) (width 2) (layer "F.Cu") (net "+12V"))
 (segment (start 96.800534 66.715) (end 86.850787 66.715) (width 2) (layer "F.Cu") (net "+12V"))
 (segment (start 95.135 90.6925) (end 95.135 96.4075) (width 2) (layer "F.Cu") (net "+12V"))
 (segment (start 95.135 79.2625) (end 98.265 76.1325) (width 2) (layer "F.Cu") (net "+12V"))
 (segment (start 95.135 79.2625) (end 95.135 85.09) (width 2) (layer "F.Cu") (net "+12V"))
 (segment (start 98.265 68.179466) (end 96.800534 66.715) (width 2) (layer "F.Cu") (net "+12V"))
 (segment (start 95.135 85.09) (end 95.135 90.6925) (width 2) (layer "F.Cu") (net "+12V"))
 (segment (start 85.765 67.800787) (end 85.765 69.215) (width 2) (layer "F.Cu") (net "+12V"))
 (segment (start 88.265 69.215) (end 88.265 72.293664) (width 1.5) (layer "F.Cu") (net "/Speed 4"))
 (segment (start 83.885 90.1575) (end 90.135 96.4075) (width 1.5) (layer "F.Cu") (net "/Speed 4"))
 (segment (start 83.885 76.673665) (end 83.885 90.1575) (width 1.5) (layer "F.Cu") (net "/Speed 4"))
 (segment (start 88.265 72.293664) (end 83.885 76.673665) (width 1.5) (layer "F.Cu") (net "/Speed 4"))
 (segment (start 86.995 56.725) (end 92.669 51.051) (width 0.5) (layer "F.Cu") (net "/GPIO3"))
 (segment (start 104.3681 51.051) (end 106.6806 53.3635) (width 0.5) (layer "F.Cu") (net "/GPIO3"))
 (segment (start 92.669 51.051) (end 104.3681 51.051) (width 0.5) (layer "F.Cu") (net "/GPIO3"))
 (segment (start 108.585 60.96) (end 106.6806 59.0556) (width 0.5) (layer "F.Cu") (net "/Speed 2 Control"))
 (segment (start 106.6806 56.2885) (end 109.2206 56.2885) (width 0.5) (layer "F.Cu") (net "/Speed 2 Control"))
 (segment (start 106.6806 59.0556) (end 106.6806 56.2885) (width 0.5) (layer "F.Cu") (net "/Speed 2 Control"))
 (segment (start 110.6031 50.051) (end 91.169 50.051) (width 0.5) (layer "F.Cu") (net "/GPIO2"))
 (segment (start 112.3956 53.3635) (end 112.3956 51.8435) (width 0.5) (layer "F.Cu") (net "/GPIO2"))
 (segment (start 91.169 50.051) (end 86.995 54.225) (width 0.5) (layer "F.Cu") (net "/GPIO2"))
 (segment (start 112.3956 51.8435) (end 110.6031 50.051) (width 0.5) (layer "F.Cu") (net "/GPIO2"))
 (segment (start 102.8281 52.051) (end 104.1406 53.3635) (width 0.5) (layer "F.Cu") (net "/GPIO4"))
 (segment (start 94.169 52.051) (end 102.8281 52.051) (width 0.5) (layer "F.Cu") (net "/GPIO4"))
 (segment (start 86.995 59.225) (end 94.169 52.051) (width 0.5) (layer "F.Cu") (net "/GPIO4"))
 (segment (start 88.745 58.889214) (end 94.164814 53.4694) (width 0.5) (layer "F.Cu") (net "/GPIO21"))
 (segment (start 86.995 61.725) (end 86.995 60.975) (width 0.5) (layer "F.Cu") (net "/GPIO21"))
 (segment (start 87.719874 60.975) (end 88.745 59.949874) (width 0.5) (layer "F.Cu") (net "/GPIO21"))
 (segment (start 94.164814 53.4694) (end 95.2506 53.4694) (width 0.5) (layer "F.Cu") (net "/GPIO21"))
 (segment (start 86.995 60.975) (end 87.719874 60.975) (width 0.5) (layer "F.Cu") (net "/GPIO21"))
 (segment (start 88.745 59.949874) (end 88.745 58.889214) (width 0.5) (layer "F.Cu") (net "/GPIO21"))
 (segment (start 103.505 60.96) (end 105.255 59.21) (width 0.5) (layer "F.Cu") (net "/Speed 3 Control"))
 (segment (start 105.255 57.4029) (end 104.1406 56.2885) (width 0.5) (layer "F.Cu") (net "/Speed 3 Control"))
 (segment (start 104.1406 56.2885) (end 101.6006 56.2885) (width 0.5) (layer "F.Cu") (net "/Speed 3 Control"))
 (segment (start 105.255 59.21) (end 105.255 57.4029) (width 0.5) (layer "F.Cu") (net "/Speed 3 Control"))
 (segment (start 111.385 90.6925) (end 103.3278 82.6353) (width 0.5) (layer "F.Cu") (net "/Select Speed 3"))
 (segment (start 103.3278 82.6353) (end 103.3278 63.6772) (width 0.5) (layer "F.Cu") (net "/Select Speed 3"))
 (segment (start 111.385 85.09) (end 104.335 78.04) (width 0.5) (layer "F.Cu") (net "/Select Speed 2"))
 (segment (start 104.335 67.440126) (end 108.275126 63.5) (width 0.5) (layer "F.Cu") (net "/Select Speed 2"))
 (segment (start 104.335 78.04) (end 104.335 67.440126) (width 0.5) (layer "F.Cu") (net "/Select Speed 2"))
 (segment (start 90.135 79.2625) (end 95.765 73.6325) (width 1.5) (layer "F.Cu") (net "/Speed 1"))
 (segment (start 95.765 73.6325) (end 95.765 69.215) (width 1.5) (layer "F.Cu") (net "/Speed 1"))
 (segment (start 115.335 75.3125) (end 115.335 64.81) (width 0.5) (layer "F.Cu") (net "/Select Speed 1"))
 (segment (start 115.335 64.81) (end 114.025 63.5) (width 0.5) (layer "F.Cu") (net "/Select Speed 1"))
 (segment (start 111.385 79.2625) (end 115.335 75.3125) (width 0.5) (layer "F.Cu") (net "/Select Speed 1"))
 (segment (start 93.265 69.215) (end 93.265 72.950519) (width 1.5) (layer "F.Cu") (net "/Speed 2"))
 (segment (start 93.265 72.950519) (end 87.885 78.330519) (width 1.5) (layer "F.Cu") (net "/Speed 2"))
 (segment (start 87.885 78.330519) (end 87.885 82.84) (width 1.5) (layer "F.Cu") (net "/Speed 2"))
 (segment (start 87.885 82.84) (end 90.135 85.09) (width 1.5) (layer "F.Cu") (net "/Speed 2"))
 (segment (start 85.885 86.4425) (end 90.135 90.6925) (width 1.5) (layer "F.Cu") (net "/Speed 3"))
 (segment (start 90.765 72.622091) (end 85.885 77.502092) (width 1.5) (layer "F.Cu") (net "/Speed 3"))
 (segment (start 90.765 69.215) (end 90.765 72.622091) (width 1.5) (layer "F.Cu") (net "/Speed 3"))
 (segment (start 85.885 77.502092) (end 85.885 86.4425) (width 1.5) (layer "F.Cu") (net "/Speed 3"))
 (segment (start 112.5226 56.2885) (end 114.9356 56.2885) (width 0.5) (layer "F.Cu") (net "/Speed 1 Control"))
 (segment (start 115.775 59.21) (end 115.775 57.1279) (width 0.5) (layer "F.Cu") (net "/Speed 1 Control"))
 (segment (start 115.775 57.1279) (end 114.9356 56.2885) (width 0.5) (layer "F.Cu") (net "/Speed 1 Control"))
 (segment (start 114.025 60.96) (end 115.775 59.21) (width 0.5) (layer "F.Cu") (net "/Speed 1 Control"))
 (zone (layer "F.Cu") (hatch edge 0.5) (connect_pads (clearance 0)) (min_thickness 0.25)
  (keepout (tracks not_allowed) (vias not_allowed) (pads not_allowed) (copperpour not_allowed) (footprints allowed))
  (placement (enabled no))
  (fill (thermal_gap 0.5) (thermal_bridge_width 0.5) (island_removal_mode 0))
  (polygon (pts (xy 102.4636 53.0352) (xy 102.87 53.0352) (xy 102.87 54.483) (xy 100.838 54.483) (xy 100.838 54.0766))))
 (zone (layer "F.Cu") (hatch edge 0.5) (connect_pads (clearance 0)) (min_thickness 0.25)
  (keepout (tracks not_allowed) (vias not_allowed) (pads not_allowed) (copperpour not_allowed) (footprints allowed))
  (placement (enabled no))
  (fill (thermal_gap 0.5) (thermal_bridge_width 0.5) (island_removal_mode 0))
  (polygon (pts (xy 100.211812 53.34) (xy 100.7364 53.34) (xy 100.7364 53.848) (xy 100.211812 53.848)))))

